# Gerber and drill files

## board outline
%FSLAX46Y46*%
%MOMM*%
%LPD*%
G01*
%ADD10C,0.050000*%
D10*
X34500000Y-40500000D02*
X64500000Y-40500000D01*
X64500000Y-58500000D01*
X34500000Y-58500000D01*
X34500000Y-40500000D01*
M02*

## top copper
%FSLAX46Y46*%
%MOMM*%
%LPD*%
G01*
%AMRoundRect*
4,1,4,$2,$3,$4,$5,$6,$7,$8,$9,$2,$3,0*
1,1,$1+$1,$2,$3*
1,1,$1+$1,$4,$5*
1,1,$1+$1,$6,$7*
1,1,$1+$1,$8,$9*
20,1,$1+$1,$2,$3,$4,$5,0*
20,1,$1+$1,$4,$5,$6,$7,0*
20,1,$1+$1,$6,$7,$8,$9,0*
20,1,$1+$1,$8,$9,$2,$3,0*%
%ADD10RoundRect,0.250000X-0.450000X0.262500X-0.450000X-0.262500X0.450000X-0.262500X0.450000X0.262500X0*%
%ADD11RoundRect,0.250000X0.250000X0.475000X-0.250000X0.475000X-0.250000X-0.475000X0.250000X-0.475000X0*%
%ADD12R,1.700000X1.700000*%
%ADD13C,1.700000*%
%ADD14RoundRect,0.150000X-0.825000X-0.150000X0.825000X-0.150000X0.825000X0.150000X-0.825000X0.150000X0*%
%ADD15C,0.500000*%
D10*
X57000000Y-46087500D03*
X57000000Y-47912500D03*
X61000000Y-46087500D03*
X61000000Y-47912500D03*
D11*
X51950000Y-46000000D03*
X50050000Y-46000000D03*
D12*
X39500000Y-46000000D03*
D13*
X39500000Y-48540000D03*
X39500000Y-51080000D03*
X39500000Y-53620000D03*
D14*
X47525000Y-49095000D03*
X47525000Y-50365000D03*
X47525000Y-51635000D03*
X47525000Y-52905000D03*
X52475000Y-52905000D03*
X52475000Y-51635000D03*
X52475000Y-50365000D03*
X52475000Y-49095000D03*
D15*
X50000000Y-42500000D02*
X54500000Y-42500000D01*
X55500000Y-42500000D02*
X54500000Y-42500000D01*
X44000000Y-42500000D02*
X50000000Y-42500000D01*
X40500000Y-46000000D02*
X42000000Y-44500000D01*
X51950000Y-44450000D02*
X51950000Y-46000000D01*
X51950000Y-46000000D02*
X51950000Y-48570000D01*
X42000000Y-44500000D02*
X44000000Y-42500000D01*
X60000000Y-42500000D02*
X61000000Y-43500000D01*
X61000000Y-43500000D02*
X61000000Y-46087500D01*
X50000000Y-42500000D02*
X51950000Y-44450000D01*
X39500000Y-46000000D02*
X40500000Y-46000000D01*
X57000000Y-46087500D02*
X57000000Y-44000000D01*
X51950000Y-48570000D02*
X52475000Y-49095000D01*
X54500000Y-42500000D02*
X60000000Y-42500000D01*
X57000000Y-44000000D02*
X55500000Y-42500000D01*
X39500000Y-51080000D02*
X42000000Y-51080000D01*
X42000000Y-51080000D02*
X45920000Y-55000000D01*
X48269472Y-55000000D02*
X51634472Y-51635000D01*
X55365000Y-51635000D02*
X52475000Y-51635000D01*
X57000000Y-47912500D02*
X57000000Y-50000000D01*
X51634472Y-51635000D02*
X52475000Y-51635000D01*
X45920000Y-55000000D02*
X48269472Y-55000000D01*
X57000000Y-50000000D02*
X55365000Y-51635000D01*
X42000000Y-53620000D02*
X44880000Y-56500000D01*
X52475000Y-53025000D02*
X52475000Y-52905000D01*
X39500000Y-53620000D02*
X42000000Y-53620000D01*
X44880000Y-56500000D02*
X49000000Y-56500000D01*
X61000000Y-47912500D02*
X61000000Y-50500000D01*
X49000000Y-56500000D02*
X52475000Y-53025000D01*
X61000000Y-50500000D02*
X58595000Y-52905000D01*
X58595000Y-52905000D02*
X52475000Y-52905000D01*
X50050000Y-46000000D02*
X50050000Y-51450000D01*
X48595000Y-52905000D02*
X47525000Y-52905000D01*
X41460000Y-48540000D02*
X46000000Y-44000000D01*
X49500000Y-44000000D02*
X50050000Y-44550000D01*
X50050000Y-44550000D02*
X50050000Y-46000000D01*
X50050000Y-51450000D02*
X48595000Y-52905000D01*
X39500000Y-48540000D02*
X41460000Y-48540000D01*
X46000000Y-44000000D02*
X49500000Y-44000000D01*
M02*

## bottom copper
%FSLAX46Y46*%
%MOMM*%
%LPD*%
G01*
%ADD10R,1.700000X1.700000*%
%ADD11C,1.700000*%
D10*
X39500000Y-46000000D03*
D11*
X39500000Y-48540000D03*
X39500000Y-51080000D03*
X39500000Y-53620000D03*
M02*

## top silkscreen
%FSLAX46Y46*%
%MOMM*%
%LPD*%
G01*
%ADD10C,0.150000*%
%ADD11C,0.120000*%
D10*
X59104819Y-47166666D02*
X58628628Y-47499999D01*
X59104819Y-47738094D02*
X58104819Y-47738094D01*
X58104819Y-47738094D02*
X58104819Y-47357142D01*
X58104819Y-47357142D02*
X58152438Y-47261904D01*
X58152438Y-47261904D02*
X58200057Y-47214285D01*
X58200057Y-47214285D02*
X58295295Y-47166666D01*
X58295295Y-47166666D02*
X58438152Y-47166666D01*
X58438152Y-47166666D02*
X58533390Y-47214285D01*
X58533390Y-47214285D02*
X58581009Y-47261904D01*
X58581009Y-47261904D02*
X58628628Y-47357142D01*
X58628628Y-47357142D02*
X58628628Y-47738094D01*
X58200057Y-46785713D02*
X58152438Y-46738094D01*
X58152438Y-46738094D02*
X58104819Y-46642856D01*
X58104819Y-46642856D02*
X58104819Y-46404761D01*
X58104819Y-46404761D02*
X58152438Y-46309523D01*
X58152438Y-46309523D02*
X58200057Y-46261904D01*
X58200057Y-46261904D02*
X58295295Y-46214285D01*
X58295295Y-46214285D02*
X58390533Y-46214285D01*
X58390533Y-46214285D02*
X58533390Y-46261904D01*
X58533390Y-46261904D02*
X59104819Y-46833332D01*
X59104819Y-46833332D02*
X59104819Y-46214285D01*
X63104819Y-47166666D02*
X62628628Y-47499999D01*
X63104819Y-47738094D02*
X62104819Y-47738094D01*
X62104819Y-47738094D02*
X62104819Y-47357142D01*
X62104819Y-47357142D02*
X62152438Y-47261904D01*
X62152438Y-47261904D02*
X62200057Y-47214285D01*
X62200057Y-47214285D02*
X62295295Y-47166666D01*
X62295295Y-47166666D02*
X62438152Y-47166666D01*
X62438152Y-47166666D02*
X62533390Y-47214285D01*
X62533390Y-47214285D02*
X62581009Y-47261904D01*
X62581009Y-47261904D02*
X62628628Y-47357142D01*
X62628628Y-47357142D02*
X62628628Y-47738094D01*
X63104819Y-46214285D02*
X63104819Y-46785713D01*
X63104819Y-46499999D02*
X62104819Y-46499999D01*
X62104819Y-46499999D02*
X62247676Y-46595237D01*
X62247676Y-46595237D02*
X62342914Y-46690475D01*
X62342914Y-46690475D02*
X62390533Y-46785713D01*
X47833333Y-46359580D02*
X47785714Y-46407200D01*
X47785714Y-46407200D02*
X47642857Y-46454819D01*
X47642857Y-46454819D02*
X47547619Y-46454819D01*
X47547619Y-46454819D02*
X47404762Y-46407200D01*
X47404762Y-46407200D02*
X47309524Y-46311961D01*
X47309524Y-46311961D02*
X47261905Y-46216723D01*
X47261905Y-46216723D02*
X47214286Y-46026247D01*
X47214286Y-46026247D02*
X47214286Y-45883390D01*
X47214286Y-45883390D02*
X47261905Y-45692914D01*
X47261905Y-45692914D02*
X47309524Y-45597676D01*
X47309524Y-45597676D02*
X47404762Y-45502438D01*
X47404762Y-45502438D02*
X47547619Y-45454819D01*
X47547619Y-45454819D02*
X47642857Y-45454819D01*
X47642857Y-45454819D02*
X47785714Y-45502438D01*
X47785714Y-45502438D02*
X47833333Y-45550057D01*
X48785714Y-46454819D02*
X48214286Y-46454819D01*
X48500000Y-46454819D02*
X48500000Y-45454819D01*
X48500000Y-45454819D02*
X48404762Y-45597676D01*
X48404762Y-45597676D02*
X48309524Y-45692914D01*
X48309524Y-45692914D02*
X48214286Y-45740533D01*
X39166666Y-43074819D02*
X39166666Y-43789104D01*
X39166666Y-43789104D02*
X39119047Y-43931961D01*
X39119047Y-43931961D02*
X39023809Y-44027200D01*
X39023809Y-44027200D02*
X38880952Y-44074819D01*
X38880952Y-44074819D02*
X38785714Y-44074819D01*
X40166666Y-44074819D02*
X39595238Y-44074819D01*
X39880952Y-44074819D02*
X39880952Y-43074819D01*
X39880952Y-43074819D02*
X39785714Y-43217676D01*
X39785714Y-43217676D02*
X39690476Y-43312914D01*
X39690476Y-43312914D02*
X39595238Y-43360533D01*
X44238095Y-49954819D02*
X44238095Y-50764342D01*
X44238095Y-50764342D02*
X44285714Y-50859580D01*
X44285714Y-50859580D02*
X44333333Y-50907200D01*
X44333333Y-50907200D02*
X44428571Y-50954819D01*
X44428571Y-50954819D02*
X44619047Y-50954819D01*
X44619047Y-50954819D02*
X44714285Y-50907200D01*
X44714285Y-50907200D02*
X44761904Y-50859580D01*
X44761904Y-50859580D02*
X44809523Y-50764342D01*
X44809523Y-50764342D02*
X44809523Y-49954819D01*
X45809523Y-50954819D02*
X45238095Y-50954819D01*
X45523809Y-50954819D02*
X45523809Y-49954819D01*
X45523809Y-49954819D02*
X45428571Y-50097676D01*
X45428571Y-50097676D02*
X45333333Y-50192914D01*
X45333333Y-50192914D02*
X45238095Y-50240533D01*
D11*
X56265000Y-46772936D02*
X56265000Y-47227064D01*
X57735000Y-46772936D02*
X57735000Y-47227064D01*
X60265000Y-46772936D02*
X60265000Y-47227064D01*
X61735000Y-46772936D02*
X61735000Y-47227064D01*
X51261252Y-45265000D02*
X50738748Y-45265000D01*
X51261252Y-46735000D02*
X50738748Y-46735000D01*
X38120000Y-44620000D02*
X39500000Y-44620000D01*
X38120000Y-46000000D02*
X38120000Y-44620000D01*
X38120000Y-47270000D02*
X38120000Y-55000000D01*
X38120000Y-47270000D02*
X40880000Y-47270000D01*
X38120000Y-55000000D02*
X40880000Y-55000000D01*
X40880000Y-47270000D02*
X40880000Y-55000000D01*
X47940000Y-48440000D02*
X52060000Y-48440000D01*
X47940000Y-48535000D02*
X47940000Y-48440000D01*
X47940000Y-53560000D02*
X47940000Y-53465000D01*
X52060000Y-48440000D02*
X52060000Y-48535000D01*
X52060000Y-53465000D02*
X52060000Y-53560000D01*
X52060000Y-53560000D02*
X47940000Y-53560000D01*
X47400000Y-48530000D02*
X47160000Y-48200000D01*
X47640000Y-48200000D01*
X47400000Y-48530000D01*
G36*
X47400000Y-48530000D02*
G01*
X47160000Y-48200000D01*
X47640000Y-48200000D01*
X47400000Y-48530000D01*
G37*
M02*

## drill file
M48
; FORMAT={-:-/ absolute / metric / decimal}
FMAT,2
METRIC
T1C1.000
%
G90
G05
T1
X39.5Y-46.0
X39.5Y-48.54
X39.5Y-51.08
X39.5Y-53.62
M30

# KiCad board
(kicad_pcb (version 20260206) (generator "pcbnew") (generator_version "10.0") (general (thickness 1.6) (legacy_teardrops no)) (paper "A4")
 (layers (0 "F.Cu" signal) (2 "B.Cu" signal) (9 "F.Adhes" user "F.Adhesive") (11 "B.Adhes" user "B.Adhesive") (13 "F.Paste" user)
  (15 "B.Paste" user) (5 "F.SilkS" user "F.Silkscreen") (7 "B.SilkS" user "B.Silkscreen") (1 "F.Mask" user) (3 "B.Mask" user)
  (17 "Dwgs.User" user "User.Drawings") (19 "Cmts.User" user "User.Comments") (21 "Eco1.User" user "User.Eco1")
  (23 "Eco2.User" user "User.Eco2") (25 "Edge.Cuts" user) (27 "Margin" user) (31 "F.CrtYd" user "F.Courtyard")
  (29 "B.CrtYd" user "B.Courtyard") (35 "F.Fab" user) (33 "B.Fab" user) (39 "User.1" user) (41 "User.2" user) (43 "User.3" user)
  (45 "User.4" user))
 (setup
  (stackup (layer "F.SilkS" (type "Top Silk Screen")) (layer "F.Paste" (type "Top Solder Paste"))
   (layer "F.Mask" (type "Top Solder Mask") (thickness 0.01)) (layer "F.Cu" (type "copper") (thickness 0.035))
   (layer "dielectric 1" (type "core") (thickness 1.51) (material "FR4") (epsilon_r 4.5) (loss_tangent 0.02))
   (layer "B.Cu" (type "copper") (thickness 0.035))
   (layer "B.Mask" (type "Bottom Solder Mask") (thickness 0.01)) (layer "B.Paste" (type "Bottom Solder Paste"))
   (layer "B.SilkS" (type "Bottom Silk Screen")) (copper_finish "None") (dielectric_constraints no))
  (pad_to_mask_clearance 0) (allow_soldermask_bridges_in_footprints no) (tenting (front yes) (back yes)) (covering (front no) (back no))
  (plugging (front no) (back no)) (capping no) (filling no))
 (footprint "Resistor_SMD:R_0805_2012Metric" (layer "F.Cu") (at 57 47 -90)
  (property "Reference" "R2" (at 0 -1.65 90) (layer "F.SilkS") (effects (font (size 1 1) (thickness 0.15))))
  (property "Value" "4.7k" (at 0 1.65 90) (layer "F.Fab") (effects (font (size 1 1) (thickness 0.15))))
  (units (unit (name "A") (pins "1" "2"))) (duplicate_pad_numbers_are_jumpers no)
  (fp_line (start -0.227064 0.735) (end 0.227064 0.735) (stroke (width 0.12) (type solid)) (layer "F.SilkS"))
  (fp_line (start -0.227064 -0.735) (end 0.227064 -0.735) (stroke (width 0.12) (type solid)) (layer "F.SilkS"))
  (pad "1" smd roundrect (at -0.9125 0 270) (size 1.025 1.4) (layers "F.Cu" "F.Mask" "F.Paste") (roundrect_rratio 0.243902) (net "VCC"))
  (pad "2" smd roundrect (at 0.9125 0 270) (size 1.025 1.4) (layers "F.Cu" "F.Mask" "F.Paste") (roundrect_rratio 0.243902)
   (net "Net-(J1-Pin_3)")))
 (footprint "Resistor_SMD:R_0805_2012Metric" (layer "F.Cu") (at 61 47 -90)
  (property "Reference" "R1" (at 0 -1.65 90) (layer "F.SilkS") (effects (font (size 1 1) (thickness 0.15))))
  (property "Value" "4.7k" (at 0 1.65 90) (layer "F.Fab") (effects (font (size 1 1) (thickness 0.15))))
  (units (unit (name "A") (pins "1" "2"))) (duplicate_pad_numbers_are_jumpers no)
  (fp_line (start -0.227064 0.735) (end 0.227064 0.735) (stroke (width 0.12) (type solid)) (layer "F.SilkS"))
  (fp_line (start -0.227064 -0.735) (end 0.227064 -0.735) (stroke (width 0.12) (type solid)) (layer "F.SilkS"))
  (pad "1" smd roundrect (at -0.9125 0 270) (size 1.025 1.4) (layers "F.Cu" "F.Mask" "F.Paste") (roundrect_rratio 0.243902) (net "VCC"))
  (pad "2" smd roundrect (at 0.9125 0 270) (size 1.025 1.4) (layers "F.Cu" "F.Mask" "F.Paste") (roundrect_rratio 0.243902)
   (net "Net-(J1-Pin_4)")))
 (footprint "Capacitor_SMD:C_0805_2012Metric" (layer "F.Cu") (at 51 46 180)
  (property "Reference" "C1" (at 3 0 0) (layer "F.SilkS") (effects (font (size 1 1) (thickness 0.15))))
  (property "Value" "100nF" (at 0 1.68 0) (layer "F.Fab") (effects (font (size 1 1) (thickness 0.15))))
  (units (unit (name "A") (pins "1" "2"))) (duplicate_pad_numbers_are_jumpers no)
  (fp_line (start -0.261252 0.735) (end 0.261252 0.735) (stroke (width 0.12) (type solid)) (layer "F.SilkS"))
  (fp_line (start -0.261252 -0.735) (end 0.261252 -0.735) (stroke (width 0.12) (type solid)) (layer "F.SilkS"))
  (pad "1" smd roundrect (at -0.95 0 180) (size 1 1.45) (layers "F.Cu" "F.Mask" "F.Paste") (roundrect_rratio 0.25) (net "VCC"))
  (pad "2" smd roundrect (at 0.95 0 180) (size 1 1.45) (layers "F.Cu" "F.Mask" "F.Paste") (roundrect_rratio 0.25) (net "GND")))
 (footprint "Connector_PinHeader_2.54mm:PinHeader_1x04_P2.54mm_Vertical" (layer "F.Cu") (at 39.5 46)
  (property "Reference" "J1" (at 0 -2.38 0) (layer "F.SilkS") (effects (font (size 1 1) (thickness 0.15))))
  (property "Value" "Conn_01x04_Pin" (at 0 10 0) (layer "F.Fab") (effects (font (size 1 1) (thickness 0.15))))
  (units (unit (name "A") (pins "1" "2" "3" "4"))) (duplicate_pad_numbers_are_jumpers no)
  (fp_line (start -1.38 -1.38) (end 0 -1.38) (stroke (width 0.12) (type solid)) (layer "F.SilkS"))
  (fp_line (start -1.38 0) (end -1.38 -1.38) (stroke (width 0.12) (type solid)) (layer "F.SilkS"))
  (fp_line (start -1.38 1.27) (end -1.38 9) (stroke (width 0.12) (type solid)) (layer "F.SilkS"))
  (fp_line (start -1.38 1.27) (end 1.38 1.27) (stroke (width 0.12) (type solid)) (layer "F.SilkS"))
  (fp_line (start -1.38 9) (end 1.38 9) (stroke (width 0.12) (type solid)) (layer "F.SilkS"))
  (fp_line (start 1.38 1.27) (end 1.38 9) (stroke (width 0.12) (type solid)) (layer "F.SilkS"))
  (pad "1" thru_hole rect (at 0 0) (size 1.7 1.7) (drill 1) (layers "*.Cu" "*.Mask") (remove_unused_layers no) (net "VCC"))
  (pad "2" thru_hole circle (at 0 2.54) (size 1.7 1.7) (drill 1) (layers "*.Cu" "*.Mask") (remove_unused_layers no) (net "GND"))
  (pad "3" thru_hole circle (at 0 5.08) (size 1.7 1.7) (drill 1) (layers "*.Cu" "*.Mask") (remove_unused_layers no) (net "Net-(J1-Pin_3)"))
  (pad "4" thru_hole circle (at 0 7.62) (size 1.7 1.7) (drill 1) (layers "*.Cu" "*.Mask") (remove_unused_layers no) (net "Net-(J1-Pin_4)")))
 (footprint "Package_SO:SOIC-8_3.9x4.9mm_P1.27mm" (layer "F.Cu") (at 50 51)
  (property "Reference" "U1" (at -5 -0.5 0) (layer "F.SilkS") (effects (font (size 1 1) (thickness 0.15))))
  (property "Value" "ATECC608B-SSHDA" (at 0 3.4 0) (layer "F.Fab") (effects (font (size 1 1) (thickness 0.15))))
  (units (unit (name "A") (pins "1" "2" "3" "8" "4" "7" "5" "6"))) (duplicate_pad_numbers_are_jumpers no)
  (fp_line (start -2.06 -2.56) (end 2.06 -2.56) (stroke (width 0.12) (type solid)) (layer "F.SilkS"))
  (fp_line (start -2.06 -2.465) (end -2.06 -2.56) (stroke (width 0.12) (type solid)) (layer "F.SilkS"))
  (fp_line (start -2.06 2.56) (end -2.06 2.465) (stroke (width 0.12) (type solid)) (layer "F.SilkS"))
  (fp_line (start 2.06 -2.56) (end 2.06 -2.465) (stroke (width 0.12) (type solid)) (layer "F.SilkS"))
  (fp_line (start 2.06 2.465) (end 2.06 2.56) (stroke (width 0.12) (type solid)) (layer "F.SilkS"))
  (fp_line (start 2.06 2.56) (end -2.06 2.56) (stroke (width 0.12) (type solid)) (layer "F.SilkS"))
  (fp_poly (pts (xy -2.6 -2.47) (xy -2.84 -2.8) (xy -2.36 -2.8)) (stroke (width 0.12) (type solid)) (fill yes) (layer "F.SilkS"))
  (pad "1" smd roundrect (at -2.475 -1.905) (size 1.95 0.6) (layers "F.Cu" "F.Mask" "F.Paste") (roundrect_rratio 0.25)
   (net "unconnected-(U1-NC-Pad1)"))
  (pad "2" smd roundrect (at -2.475 -0.635) (size 1.95 0.6) (layers "F.Cu" "F.Mask" "F.Paste") (roundrect_rratio 0.25)
   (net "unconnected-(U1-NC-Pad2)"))
  (pad "3" smd roundrect (at -2.475 0.635) (size 1.95 0.6) (layers "F.Cu" "F.Mask" "F.Paste") (roundrect_rratio 0.25)
   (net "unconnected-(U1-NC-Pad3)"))
  (pad "4" smd roundrect (at -2.475 1.905) (size 1.95 0.6) (layers "F.Cu" "F.Mask" "F.Paste") (roundrect_rratio 0.25) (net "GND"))
  (pad "5" smd roundrect (at 2.475 1.905) (size 1.95 0.6) (layers "F.Cu" "F.Mask" "F.Paste") (roundrect_rratio 0.25) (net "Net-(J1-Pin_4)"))
  (pad "6" smd roundrect (at 2.475 0.635) (size 1.95 0.6) (layers "F.Cu" "F.Mask" "F.Paste") (roundrect_rratio 0.25) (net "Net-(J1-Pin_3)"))
  (pad "7" smd roundrect (at 2.475 -0.635) (size 1.95 0.6) (layers "F.Cu" "F.Mask" "F.Paste") (roundrect_rratio 0.25)
   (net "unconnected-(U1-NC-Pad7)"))
  (pad "8" smd roundrect (at 2.475 -1.905) (size 1.95 0.6) (layers "F.Cu" "F.Mask" "F.Paste") (roundrect_rratio 0.25) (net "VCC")))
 (gr_rect (start 34.5 40.5) (end 64.5 58.5) (stroke (width 0.05) (type default)) (fill no) (layer "Edge.Cuts"))
 (segment (start 50 42.5) (end 54.5 42.5) (width 0.5) (layer "F.Cu") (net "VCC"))
 (segment (start 55.5 42.5) (end 54.5 42.5) (width 0.5) (layer "F.Cu") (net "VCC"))
 (segment (start 44 42.5) (end 50 42.5) (width 0.5) (layer "F.Cu") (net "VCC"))
 (segment (start 40.5 46) (end 42 44.5) (width 0.5) (layer "F.Cu") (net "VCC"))
 (segment (start 51.95 44.45) (end 51.95 46) (width 0.5) (layer "F.Cu") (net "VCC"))
 (segment (start 51.95 46) (end 51.95 48.57) (width 0.5) (layer "F.Cu") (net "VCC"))
 (segment (start 42 44.5) (end 44 42.5) (width 0.5) (layer "F.Cu") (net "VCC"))
 (segment (start 60 42.5) (end 61 43.5) (width 0.5) (layer "F.Cu") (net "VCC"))
 (segment (start 61 43.5) (end 61 46.0875) (width 0.5) (layer "F.Cu") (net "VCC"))
 (segment (start 50 42.5) (end 51.95 44.45) (width 0.5) (layer "F.Cu") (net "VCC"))
 (segment (start 39.5 46) (end 40.5 46) (width 0.5) (layer "F.Cu") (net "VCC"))
 (segment (start 57 46.0875) (end 57 44) (width 0.5) (layer "F.Cu") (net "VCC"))
 (segment (start 51.95 48.57) (end 52.475 49.095) (width 0.5) (layer "F.Cu") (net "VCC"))
 (segment (start 54.5 42.5) (end 60 42.5) (width 0.5) (layer "F.Cu") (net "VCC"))
 (segment (start 57 44) (end 55.5 42.5) (width 0.5) (layer "F.Cu") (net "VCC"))
 (segment (start 39.5 51.08) (end 42 51.08) (width 0.5) (layer "F.Cu") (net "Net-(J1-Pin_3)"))
 (segment (start 42 51.08) (end 45.92 55) (width 0.5) (layer "F.Cu") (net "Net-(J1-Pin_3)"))
 (segment (start 48.269472 55) (end 51.634472 51.635) (width 0.5) (layer "F.Cu") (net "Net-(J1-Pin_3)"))
 (segment (start 55.365 51.635) (end 52.475 51.635) (width 0.5) (layer "F.Cu") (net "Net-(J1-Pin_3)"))
 (segment (start 57 47.9125) (end 57 50) (width 0.5) (layer "F.Cu") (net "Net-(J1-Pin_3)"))
 (segment (start 51.634472 51.635) (end 52.475 51.635) (width 0.5) (layer "F.Cu") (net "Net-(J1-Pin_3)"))
 (segment (start 45.92 55) (end 48.269472 55) (width 0.5) (layer "F.Cu") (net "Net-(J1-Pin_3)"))
 (segment (start 57 50) (end 55.365 51.635) (width 0.5) (layer "F.Cu") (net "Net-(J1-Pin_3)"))
 (segment (start 42 53.62) (end 44.88 56.5) (width 0.5) (layer "F.Cu") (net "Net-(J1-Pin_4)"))
 (segment (start 52.475 53.025) (end 52.475 52.905) (width 0.5) (layer "F.Cu") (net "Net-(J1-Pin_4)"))
 (segment (start 39.5 53.62) (end 42 53.62) (width 0.5) (layer "F.Cu") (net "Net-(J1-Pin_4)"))
 (segment (start 44.88 56.5) (end 49 56.5) (width 0.5) (layer "F.Cu") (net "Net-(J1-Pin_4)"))
 (segment (start 61 47.9125) (end 61 50.5) (width 0.5) (layer "F.Cu") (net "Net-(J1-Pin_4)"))
 (segment (start 49 56.5) (end 52.475 53.025) (width 0.5) (layer "F.Cu") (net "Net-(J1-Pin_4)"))
 (segment (start 61 50.5) (end 58.595 52.905) (width 0.5) (layer "F.Cu") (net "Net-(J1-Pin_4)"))
 (segment (start 58.595 52.905) (end 52.475 52.905) (width 0.5) (layer "F.Cu") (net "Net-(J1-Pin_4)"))
 (segment (start 50.05 46) (end 50.05 51.45) (width 0.5) (layer "F.Cu") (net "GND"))
 (segment (start 48.595 52.905) (end 47.525 52.905) (width 0.5) (layer "F.Cu") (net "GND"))
 (segment (start 41.46 48.54) (end 46 44) (width 0.5) (layer "F.Cu") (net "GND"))
 (segment (start 49.5 44) (end 50.05 44.55) (width 0.5) (layer "F.Cu") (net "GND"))
 (segment (start 50.05 44.55) (end 50.05 46) (width 0.5) (layer "F.Cu") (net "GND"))
 (segment (start 50.05 51.45) (end 48.595 52.905) (width 0.5) (layer "F.Cu") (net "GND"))
 (segment (start 39.5 48.54) (end 41.46 48.54) (width 0.5) (layer "F.Cu") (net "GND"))
 (segment (start 46 44) (end 49.5 44) (width 0.5) (layer "F.Cu") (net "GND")))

